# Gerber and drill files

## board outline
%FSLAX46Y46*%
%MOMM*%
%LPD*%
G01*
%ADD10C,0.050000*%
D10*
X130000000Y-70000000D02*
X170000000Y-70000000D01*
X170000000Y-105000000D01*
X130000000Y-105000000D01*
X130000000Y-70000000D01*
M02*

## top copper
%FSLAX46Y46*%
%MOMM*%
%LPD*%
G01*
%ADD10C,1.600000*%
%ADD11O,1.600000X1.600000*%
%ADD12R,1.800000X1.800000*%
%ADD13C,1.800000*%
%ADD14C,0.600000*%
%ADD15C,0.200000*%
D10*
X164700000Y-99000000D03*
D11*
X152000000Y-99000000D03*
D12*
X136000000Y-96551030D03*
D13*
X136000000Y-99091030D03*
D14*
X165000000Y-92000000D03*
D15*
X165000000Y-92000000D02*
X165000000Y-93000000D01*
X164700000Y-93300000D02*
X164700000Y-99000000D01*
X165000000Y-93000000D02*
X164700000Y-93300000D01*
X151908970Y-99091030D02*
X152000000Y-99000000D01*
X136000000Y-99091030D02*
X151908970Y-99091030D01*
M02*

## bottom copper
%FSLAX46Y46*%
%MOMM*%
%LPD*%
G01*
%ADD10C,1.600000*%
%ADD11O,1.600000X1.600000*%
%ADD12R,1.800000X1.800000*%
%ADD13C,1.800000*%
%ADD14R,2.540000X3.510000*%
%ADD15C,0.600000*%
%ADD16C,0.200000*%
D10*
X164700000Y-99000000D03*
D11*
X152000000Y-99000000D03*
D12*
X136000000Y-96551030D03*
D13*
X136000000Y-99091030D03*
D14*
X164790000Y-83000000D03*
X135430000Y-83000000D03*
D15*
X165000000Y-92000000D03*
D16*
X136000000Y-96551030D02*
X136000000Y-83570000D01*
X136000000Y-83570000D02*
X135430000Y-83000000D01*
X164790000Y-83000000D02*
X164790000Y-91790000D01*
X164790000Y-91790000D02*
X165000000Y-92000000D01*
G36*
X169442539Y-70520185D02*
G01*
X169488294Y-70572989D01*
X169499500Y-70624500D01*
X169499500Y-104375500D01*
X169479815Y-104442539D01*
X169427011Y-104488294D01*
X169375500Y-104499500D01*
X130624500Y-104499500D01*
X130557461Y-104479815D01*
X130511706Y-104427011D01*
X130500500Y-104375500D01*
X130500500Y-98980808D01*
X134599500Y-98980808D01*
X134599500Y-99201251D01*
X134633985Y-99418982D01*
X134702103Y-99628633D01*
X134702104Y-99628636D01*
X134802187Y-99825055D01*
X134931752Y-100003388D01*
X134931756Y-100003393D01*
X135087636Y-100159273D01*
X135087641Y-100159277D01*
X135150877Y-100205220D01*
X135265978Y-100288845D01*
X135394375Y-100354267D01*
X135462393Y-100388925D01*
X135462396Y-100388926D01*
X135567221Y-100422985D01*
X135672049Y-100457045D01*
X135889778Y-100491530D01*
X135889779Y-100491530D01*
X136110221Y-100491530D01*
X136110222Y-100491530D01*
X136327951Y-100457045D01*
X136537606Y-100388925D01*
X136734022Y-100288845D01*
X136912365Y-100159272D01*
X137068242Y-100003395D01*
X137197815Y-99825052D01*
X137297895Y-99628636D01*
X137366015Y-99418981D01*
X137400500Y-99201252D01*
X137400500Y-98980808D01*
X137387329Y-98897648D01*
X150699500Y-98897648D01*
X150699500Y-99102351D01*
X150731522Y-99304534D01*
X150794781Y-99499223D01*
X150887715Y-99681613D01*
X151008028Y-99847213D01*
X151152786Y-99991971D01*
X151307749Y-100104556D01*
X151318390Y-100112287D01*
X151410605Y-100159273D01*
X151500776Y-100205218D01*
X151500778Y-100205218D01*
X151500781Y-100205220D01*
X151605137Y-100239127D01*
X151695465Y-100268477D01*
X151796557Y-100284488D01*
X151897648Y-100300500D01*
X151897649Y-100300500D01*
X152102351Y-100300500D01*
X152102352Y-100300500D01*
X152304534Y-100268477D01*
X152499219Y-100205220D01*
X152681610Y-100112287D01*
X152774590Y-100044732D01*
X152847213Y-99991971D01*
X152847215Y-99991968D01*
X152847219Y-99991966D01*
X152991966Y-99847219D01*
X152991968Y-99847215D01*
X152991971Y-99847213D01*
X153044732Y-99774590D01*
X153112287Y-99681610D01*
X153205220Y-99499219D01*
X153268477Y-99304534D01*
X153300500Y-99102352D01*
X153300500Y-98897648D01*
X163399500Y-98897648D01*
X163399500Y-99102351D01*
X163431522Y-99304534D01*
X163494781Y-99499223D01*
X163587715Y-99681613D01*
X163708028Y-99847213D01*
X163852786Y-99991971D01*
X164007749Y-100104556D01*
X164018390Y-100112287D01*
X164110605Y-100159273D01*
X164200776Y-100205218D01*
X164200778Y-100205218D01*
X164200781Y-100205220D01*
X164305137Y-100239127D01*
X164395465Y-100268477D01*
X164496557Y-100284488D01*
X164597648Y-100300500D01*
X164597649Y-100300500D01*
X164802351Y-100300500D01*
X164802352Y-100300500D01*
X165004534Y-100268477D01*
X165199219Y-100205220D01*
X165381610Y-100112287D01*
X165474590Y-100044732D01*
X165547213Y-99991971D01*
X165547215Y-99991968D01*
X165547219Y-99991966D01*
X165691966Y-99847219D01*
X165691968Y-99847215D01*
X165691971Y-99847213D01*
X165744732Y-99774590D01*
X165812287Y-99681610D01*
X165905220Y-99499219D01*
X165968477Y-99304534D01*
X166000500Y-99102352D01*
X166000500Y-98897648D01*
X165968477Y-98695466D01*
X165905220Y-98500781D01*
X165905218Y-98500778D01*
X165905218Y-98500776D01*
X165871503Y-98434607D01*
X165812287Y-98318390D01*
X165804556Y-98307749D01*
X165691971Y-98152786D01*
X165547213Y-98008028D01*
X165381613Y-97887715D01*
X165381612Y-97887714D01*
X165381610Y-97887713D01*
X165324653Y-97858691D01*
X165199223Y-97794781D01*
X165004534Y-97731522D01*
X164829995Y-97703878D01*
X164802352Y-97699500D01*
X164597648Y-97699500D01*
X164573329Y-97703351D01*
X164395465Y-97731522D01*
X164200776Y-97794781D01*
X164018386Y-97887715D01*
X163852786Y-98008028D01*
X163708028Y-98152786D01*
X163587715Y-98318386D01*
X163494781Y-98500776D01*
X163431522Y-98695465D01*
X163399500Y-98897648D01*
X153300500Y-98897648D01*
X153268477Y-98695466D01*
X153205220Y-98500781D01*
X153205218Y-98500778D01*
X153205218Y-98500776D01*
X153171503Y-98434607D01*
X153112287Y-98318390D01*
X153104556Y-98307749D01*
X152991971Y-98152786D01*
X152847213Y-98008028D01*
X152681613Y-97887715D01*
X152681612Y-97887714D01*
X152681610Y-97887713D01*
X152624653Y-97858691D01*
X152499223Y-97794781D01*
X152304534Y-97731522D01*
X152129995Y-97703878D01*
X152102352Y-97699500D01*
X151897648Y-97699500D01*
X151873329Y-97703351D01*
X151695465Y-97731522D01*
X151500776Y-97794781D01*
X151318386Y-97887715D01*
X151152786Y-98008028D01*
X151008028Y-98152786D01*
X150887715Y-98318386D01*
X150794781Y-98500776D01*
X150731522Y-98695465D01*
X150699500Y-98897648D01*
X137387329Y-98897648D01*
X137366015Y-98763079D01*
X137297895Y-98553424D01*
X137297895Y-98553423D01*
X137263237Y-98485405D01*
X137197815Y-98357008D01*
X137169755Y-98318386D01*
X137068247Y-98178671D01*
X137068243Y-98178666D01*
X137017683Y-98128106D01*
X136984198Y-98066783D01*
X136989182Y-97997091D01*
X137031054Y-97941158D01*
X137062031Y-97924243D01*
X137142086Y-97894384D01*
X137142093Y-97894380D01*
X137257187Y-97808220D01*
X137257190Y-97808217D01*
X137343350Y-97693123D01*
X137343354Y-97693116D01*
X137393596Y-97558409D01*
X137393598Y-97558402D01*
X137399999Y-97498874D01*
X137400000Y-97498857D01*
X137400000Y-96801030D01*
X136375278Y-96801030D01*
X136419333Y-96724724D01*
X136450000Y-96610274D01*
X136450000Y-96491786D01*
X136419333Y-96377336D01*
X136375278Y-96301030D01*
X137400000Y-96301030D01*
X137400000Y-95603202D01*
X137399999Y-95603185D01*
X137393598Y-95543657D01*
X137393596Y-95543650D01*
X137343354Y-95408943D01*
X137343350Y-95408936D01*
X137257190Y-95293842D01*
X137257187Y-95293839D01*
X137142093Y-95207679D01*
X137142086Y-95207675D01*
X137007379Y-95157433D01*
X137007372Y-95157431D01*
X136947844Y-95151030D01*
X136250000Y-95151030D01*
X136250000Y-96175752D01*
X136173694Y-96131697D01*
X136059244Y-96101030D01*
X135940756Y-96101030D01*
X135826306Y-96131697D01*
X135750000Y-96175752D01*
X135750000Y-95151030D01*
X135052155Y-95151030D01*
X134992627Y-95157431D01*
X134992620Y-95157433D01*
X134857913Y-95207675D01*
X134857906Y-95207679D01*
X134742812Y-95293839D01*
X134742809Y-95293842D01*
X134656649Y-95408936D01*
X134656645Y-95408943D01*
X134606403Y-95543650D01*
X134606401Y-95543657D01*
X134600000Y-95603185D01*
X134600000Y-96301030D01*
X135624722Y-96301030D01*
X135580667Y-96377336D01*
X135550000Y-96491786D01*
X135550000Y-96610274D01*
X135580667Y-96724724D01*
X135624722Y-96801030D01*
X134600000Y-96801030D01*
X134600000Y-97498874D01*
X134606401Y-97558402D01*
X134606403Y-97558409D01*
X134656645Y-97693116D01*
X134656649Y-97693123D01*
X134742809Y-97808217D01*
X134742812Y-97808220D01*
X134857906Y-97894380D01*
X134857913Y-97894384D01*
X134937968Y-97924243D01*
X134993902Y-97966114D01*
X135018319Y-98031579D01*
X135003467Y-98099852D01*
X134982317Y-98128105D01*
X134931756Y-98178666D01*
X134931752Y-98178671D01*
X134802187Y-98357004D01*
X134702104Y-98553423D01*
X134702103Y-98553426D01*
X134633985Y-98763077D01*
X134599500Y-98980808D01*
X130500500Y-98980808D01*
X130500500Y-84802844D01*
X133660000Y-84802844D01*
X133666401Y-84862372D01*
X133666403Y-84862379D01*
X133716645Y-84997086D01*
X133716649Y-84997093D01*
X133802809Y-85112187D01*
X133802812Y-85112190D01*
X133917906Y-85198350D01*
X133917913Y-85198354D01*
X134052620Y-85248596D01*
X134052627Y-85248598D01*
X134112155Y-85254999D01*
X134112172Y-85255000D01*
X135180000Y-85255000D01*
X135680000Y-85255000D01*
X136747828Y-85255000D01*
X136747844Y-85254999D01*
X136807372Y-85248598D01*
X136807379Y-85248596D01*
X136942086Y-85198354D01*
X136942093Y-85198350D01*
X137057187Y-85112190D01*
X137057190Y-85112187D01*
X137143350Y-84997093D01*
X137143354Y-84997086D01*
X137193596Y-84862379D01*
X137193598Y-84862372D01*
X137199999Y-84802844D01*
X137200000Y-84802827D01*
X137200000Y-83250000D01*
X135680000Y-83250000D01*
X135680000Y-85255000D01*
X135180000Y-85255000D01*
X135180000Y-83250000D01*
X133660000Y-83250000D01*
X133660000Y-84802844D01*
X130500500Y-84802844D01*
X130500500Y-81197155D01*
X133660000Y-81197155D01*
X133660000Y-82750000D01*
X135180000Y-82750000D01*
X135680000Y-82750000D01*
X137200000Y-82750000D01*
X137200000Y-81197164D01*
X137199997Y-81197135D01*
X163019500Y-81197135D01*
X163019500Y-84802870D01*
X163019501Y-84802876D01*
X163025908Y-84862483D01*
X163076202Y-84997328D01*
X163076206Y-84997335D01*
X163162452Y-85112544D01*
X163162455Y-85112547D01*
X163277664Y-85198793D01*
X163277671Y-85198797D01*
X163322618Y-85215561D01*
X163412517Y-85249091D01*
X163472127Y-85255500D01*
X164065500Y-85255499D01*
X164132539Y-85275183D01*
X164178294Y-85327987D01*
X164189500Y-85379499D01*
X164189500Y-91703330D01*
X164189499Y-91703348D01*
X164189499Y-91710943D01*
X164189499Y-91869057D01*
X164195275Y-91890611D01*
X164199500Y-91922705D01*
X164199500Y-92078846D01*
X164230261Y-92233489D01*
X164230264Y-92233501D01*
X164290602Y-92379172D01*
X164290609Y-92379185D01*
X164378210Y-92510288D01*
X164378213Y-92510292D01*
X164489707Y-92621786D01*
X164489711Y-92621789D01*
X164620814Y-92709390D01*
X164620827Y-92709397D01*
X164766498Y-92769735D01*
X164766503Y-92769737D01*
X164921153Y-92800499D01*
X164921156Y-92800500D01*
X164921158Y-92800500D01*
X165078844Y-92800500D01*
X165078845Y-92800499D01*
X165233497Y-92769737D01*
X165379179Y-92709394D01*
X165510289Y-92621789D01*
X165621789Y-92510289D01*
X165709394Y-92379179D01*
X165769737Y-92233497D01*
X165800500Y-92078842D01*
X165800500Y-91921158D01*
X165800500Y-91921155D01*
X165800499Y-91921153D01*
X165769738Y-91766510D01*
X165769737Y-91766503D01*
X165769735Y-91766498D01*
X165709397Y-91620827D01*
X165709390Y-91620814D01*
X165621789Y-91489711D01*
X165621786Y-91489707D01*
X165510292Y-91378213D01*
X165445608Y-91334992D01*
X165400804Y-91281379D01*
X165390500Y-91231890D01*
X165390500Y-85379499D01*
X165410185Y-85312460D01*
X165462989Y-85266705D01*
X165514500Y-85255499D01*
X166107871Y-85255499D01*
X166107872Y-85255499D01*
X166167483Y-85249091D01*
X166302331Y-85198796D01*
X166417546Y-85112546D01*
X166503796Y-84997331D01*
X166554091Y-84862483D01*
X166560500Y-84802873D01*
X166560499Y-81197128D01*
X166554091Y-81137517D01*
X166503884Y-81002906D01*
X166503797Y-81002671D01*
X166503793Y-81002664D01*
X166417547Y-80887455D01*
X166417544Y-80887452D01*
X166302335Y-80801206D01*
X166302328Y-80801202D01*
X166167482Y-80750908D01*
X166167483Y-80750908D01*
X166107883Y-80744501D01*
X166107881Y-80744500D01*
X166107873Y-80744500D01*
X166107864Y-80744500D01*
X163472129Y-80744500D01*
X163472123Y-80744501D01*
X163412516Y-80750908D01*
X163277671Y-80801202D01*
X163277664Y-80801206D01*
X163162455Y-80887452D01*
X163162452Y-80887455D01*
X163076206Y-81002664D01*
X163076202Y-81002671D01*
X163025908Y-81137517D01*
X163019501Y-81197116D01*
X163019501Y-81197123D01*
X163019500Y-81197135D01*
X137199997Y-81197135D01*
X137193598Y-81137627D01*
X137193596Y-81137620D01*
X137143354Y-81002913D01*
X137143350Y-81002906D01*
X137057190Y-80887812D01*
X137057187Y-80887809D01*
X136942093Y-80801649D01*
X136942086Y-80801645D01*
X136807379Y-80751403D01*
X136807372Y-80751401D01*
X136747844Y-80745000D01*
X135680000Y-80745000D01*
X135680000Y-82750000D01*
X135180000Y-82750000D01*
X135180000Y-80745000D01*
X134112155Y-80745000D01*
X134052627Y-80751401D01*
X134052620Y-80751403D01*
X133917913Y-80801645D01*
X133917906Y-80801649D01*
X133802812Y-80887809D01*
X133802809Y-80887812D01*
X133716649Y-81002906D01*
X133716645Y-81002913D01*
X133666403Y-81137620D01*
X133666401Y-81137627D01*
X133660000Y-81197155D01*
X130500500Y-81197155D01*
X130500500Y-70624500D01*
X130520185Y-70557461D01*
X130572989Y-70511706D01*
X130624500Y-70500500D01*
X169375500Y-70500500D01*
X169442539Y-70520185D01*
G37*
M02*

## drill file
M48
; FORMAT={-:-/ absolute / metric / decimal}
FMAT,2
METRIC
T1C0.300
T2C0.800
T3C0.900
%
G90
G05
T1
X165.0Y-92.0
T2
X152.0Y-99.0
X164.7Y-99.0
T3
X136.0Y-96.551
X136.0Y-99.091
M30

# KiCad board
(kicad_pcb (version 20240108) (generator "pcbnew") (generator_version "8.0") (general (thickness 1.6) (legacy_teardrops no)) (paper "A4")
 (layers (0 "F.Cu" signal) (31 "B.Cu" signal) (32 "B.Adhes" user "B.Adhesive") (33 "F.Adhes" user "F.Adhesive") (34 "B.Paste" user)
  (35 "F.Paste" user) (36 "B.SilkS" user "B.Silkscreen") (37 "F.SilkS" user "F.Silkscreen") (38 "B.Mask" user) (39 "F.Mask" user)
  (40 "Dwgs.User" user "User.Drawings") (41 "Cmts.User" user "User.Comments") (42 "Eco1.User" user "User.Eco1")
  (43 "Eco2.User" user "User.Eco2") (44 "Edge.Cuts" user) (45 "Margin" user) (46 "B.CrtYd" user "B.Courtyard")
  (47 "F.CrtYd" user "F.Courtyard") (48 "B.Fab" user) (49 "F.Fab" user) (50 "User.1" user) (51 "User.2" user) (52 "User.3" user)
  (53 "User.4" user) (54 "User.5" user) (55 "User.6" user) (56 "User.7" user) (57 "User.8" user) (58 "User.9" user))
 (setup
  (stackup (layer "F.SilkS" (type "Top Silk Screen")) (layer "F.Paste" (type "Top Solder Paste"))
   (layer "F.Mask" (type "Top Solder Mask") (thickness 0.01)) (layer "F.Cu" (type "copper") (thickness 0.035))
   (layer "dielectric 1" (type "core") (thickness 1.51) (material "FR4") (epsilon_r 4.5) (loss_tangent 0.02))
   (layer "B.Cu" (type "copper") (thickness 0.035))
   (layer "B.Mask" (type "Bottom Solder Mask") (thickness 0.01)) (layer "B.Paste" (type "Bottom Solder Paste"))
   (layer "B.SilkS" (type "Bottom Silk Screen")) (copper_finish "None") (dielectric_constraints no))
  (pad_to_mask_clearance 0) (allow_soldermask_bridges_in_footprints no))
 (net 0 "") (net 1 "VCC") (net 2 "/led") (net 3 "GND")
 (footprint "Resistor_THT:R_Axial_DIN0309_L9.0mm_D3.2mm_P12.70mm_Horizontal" (layer "F.Cu") (at 164.7 99 180)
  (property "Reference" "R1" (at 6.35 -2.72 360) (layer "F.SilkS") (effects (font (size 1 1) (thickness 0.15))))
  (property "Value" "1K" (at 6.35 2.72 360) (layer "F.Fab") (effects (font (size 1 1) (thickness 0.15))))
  (pad "1" thru_hole circle (at 0 0 180) (size 1.6 1.6) (drill 0.8) (layers "*.Cu" "*.Mask") (remove_unused_layers no) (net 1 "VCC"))
  (pad "2" thru_hole oval (at 12.7 0 180) (size 1.6 1.6) (drill 0.8) (layers "*.Cu" "*.Mask") (remove_unused_layers no) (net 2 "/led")))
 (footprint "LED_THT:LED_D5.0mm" (layer "F.Cu") (at 136 96.55103 -90)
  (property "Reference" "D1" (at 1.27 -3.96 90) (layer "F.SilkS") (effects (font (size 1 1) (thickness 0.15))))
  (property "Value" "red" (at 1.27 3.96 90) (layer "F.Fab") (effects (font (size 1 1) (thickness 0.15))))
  (pad "1" thru_hole rect (at 0 0 270) (size 1.8 1.8) (drill 0.9) (layers "*.Cu" "*.Mask") (remove_unused_layers no) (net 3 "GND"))
  (pad "2" thru_hole circle (at 2.54 0 270) (size 1.8 1.8) (drill 0.9) (layers "*.Cu" "*.Mask") (remove_unused_layers no) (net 2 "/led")))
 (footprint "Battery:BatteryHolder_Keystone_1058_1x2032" (layer "B.Cu") (at 150.11 83 180)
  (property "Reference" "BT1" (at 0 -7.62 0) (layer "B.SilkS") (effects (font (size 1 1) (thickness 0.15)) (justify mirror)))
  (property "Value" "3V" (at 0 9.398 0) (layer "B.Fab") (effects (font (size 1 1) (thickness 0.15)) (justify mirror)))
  (pad "1" smd rect (at -14.68 0 180) (size 2.54 3.51) (layers "B.Cu" "B.Paste" "B.Mask") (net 1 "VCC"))
  (pad "2" smd rect (at 14.68 0 180) (size 2.54 3.51) (layers "B.Cu" "B.Paste" "B.Mask") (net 3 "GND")))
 (gr_rect (start 130 70) (end 170 105) (stroke (width 0.05) (type default)) (fill none) (layer "Edge.Cuts"))
 (segment (start 136 96.55103) (end 136 83.57) (width 0.2) (layer "B.Cu") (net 3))
 (segment (start 136 83.57) (end 135.43 83) (width 0.2) (layer "B.Cu") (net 3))
 (segment (start 165 92) (end 165 93) (width 0.2) (layer "F.Cu") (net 1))
 (segment (start 164.7 93.3) (end 164.7 99) (width 0.2) (layer "F.Cu") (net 1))
 (segment (start 165 93) (end 164.7 93.3) (width 0.2) (layer "F.Cu") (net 1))
 (via (at 165 92) (size 0.6) (drill 0.3) (layers "F.Cu" "B.Cu") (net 1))
 (segment (start 164.79 83) (end 164.79 91.79) (width 0.2) (layer "B.Cu") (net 1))
 (segment (start 164.79 91.79) (end 165 92) (width 0.2) (layer "B.Cu") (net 1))
 (segment (start 151.90897 99.09103) (end 152 99) (width 0.2) (layer "F.Cu") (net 2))
 (segment (start 136 99.09103) (end 151.90897 99.09103) (width 0.2) (layer "F.Cu") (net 2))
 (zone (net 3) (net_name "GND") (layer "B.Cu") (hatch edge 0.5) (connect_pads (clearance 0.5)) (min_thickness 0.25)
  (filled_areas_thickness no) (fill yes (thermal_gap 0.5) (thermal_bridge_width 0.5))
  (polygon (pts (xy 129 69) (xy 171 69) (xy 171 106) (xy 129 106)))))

